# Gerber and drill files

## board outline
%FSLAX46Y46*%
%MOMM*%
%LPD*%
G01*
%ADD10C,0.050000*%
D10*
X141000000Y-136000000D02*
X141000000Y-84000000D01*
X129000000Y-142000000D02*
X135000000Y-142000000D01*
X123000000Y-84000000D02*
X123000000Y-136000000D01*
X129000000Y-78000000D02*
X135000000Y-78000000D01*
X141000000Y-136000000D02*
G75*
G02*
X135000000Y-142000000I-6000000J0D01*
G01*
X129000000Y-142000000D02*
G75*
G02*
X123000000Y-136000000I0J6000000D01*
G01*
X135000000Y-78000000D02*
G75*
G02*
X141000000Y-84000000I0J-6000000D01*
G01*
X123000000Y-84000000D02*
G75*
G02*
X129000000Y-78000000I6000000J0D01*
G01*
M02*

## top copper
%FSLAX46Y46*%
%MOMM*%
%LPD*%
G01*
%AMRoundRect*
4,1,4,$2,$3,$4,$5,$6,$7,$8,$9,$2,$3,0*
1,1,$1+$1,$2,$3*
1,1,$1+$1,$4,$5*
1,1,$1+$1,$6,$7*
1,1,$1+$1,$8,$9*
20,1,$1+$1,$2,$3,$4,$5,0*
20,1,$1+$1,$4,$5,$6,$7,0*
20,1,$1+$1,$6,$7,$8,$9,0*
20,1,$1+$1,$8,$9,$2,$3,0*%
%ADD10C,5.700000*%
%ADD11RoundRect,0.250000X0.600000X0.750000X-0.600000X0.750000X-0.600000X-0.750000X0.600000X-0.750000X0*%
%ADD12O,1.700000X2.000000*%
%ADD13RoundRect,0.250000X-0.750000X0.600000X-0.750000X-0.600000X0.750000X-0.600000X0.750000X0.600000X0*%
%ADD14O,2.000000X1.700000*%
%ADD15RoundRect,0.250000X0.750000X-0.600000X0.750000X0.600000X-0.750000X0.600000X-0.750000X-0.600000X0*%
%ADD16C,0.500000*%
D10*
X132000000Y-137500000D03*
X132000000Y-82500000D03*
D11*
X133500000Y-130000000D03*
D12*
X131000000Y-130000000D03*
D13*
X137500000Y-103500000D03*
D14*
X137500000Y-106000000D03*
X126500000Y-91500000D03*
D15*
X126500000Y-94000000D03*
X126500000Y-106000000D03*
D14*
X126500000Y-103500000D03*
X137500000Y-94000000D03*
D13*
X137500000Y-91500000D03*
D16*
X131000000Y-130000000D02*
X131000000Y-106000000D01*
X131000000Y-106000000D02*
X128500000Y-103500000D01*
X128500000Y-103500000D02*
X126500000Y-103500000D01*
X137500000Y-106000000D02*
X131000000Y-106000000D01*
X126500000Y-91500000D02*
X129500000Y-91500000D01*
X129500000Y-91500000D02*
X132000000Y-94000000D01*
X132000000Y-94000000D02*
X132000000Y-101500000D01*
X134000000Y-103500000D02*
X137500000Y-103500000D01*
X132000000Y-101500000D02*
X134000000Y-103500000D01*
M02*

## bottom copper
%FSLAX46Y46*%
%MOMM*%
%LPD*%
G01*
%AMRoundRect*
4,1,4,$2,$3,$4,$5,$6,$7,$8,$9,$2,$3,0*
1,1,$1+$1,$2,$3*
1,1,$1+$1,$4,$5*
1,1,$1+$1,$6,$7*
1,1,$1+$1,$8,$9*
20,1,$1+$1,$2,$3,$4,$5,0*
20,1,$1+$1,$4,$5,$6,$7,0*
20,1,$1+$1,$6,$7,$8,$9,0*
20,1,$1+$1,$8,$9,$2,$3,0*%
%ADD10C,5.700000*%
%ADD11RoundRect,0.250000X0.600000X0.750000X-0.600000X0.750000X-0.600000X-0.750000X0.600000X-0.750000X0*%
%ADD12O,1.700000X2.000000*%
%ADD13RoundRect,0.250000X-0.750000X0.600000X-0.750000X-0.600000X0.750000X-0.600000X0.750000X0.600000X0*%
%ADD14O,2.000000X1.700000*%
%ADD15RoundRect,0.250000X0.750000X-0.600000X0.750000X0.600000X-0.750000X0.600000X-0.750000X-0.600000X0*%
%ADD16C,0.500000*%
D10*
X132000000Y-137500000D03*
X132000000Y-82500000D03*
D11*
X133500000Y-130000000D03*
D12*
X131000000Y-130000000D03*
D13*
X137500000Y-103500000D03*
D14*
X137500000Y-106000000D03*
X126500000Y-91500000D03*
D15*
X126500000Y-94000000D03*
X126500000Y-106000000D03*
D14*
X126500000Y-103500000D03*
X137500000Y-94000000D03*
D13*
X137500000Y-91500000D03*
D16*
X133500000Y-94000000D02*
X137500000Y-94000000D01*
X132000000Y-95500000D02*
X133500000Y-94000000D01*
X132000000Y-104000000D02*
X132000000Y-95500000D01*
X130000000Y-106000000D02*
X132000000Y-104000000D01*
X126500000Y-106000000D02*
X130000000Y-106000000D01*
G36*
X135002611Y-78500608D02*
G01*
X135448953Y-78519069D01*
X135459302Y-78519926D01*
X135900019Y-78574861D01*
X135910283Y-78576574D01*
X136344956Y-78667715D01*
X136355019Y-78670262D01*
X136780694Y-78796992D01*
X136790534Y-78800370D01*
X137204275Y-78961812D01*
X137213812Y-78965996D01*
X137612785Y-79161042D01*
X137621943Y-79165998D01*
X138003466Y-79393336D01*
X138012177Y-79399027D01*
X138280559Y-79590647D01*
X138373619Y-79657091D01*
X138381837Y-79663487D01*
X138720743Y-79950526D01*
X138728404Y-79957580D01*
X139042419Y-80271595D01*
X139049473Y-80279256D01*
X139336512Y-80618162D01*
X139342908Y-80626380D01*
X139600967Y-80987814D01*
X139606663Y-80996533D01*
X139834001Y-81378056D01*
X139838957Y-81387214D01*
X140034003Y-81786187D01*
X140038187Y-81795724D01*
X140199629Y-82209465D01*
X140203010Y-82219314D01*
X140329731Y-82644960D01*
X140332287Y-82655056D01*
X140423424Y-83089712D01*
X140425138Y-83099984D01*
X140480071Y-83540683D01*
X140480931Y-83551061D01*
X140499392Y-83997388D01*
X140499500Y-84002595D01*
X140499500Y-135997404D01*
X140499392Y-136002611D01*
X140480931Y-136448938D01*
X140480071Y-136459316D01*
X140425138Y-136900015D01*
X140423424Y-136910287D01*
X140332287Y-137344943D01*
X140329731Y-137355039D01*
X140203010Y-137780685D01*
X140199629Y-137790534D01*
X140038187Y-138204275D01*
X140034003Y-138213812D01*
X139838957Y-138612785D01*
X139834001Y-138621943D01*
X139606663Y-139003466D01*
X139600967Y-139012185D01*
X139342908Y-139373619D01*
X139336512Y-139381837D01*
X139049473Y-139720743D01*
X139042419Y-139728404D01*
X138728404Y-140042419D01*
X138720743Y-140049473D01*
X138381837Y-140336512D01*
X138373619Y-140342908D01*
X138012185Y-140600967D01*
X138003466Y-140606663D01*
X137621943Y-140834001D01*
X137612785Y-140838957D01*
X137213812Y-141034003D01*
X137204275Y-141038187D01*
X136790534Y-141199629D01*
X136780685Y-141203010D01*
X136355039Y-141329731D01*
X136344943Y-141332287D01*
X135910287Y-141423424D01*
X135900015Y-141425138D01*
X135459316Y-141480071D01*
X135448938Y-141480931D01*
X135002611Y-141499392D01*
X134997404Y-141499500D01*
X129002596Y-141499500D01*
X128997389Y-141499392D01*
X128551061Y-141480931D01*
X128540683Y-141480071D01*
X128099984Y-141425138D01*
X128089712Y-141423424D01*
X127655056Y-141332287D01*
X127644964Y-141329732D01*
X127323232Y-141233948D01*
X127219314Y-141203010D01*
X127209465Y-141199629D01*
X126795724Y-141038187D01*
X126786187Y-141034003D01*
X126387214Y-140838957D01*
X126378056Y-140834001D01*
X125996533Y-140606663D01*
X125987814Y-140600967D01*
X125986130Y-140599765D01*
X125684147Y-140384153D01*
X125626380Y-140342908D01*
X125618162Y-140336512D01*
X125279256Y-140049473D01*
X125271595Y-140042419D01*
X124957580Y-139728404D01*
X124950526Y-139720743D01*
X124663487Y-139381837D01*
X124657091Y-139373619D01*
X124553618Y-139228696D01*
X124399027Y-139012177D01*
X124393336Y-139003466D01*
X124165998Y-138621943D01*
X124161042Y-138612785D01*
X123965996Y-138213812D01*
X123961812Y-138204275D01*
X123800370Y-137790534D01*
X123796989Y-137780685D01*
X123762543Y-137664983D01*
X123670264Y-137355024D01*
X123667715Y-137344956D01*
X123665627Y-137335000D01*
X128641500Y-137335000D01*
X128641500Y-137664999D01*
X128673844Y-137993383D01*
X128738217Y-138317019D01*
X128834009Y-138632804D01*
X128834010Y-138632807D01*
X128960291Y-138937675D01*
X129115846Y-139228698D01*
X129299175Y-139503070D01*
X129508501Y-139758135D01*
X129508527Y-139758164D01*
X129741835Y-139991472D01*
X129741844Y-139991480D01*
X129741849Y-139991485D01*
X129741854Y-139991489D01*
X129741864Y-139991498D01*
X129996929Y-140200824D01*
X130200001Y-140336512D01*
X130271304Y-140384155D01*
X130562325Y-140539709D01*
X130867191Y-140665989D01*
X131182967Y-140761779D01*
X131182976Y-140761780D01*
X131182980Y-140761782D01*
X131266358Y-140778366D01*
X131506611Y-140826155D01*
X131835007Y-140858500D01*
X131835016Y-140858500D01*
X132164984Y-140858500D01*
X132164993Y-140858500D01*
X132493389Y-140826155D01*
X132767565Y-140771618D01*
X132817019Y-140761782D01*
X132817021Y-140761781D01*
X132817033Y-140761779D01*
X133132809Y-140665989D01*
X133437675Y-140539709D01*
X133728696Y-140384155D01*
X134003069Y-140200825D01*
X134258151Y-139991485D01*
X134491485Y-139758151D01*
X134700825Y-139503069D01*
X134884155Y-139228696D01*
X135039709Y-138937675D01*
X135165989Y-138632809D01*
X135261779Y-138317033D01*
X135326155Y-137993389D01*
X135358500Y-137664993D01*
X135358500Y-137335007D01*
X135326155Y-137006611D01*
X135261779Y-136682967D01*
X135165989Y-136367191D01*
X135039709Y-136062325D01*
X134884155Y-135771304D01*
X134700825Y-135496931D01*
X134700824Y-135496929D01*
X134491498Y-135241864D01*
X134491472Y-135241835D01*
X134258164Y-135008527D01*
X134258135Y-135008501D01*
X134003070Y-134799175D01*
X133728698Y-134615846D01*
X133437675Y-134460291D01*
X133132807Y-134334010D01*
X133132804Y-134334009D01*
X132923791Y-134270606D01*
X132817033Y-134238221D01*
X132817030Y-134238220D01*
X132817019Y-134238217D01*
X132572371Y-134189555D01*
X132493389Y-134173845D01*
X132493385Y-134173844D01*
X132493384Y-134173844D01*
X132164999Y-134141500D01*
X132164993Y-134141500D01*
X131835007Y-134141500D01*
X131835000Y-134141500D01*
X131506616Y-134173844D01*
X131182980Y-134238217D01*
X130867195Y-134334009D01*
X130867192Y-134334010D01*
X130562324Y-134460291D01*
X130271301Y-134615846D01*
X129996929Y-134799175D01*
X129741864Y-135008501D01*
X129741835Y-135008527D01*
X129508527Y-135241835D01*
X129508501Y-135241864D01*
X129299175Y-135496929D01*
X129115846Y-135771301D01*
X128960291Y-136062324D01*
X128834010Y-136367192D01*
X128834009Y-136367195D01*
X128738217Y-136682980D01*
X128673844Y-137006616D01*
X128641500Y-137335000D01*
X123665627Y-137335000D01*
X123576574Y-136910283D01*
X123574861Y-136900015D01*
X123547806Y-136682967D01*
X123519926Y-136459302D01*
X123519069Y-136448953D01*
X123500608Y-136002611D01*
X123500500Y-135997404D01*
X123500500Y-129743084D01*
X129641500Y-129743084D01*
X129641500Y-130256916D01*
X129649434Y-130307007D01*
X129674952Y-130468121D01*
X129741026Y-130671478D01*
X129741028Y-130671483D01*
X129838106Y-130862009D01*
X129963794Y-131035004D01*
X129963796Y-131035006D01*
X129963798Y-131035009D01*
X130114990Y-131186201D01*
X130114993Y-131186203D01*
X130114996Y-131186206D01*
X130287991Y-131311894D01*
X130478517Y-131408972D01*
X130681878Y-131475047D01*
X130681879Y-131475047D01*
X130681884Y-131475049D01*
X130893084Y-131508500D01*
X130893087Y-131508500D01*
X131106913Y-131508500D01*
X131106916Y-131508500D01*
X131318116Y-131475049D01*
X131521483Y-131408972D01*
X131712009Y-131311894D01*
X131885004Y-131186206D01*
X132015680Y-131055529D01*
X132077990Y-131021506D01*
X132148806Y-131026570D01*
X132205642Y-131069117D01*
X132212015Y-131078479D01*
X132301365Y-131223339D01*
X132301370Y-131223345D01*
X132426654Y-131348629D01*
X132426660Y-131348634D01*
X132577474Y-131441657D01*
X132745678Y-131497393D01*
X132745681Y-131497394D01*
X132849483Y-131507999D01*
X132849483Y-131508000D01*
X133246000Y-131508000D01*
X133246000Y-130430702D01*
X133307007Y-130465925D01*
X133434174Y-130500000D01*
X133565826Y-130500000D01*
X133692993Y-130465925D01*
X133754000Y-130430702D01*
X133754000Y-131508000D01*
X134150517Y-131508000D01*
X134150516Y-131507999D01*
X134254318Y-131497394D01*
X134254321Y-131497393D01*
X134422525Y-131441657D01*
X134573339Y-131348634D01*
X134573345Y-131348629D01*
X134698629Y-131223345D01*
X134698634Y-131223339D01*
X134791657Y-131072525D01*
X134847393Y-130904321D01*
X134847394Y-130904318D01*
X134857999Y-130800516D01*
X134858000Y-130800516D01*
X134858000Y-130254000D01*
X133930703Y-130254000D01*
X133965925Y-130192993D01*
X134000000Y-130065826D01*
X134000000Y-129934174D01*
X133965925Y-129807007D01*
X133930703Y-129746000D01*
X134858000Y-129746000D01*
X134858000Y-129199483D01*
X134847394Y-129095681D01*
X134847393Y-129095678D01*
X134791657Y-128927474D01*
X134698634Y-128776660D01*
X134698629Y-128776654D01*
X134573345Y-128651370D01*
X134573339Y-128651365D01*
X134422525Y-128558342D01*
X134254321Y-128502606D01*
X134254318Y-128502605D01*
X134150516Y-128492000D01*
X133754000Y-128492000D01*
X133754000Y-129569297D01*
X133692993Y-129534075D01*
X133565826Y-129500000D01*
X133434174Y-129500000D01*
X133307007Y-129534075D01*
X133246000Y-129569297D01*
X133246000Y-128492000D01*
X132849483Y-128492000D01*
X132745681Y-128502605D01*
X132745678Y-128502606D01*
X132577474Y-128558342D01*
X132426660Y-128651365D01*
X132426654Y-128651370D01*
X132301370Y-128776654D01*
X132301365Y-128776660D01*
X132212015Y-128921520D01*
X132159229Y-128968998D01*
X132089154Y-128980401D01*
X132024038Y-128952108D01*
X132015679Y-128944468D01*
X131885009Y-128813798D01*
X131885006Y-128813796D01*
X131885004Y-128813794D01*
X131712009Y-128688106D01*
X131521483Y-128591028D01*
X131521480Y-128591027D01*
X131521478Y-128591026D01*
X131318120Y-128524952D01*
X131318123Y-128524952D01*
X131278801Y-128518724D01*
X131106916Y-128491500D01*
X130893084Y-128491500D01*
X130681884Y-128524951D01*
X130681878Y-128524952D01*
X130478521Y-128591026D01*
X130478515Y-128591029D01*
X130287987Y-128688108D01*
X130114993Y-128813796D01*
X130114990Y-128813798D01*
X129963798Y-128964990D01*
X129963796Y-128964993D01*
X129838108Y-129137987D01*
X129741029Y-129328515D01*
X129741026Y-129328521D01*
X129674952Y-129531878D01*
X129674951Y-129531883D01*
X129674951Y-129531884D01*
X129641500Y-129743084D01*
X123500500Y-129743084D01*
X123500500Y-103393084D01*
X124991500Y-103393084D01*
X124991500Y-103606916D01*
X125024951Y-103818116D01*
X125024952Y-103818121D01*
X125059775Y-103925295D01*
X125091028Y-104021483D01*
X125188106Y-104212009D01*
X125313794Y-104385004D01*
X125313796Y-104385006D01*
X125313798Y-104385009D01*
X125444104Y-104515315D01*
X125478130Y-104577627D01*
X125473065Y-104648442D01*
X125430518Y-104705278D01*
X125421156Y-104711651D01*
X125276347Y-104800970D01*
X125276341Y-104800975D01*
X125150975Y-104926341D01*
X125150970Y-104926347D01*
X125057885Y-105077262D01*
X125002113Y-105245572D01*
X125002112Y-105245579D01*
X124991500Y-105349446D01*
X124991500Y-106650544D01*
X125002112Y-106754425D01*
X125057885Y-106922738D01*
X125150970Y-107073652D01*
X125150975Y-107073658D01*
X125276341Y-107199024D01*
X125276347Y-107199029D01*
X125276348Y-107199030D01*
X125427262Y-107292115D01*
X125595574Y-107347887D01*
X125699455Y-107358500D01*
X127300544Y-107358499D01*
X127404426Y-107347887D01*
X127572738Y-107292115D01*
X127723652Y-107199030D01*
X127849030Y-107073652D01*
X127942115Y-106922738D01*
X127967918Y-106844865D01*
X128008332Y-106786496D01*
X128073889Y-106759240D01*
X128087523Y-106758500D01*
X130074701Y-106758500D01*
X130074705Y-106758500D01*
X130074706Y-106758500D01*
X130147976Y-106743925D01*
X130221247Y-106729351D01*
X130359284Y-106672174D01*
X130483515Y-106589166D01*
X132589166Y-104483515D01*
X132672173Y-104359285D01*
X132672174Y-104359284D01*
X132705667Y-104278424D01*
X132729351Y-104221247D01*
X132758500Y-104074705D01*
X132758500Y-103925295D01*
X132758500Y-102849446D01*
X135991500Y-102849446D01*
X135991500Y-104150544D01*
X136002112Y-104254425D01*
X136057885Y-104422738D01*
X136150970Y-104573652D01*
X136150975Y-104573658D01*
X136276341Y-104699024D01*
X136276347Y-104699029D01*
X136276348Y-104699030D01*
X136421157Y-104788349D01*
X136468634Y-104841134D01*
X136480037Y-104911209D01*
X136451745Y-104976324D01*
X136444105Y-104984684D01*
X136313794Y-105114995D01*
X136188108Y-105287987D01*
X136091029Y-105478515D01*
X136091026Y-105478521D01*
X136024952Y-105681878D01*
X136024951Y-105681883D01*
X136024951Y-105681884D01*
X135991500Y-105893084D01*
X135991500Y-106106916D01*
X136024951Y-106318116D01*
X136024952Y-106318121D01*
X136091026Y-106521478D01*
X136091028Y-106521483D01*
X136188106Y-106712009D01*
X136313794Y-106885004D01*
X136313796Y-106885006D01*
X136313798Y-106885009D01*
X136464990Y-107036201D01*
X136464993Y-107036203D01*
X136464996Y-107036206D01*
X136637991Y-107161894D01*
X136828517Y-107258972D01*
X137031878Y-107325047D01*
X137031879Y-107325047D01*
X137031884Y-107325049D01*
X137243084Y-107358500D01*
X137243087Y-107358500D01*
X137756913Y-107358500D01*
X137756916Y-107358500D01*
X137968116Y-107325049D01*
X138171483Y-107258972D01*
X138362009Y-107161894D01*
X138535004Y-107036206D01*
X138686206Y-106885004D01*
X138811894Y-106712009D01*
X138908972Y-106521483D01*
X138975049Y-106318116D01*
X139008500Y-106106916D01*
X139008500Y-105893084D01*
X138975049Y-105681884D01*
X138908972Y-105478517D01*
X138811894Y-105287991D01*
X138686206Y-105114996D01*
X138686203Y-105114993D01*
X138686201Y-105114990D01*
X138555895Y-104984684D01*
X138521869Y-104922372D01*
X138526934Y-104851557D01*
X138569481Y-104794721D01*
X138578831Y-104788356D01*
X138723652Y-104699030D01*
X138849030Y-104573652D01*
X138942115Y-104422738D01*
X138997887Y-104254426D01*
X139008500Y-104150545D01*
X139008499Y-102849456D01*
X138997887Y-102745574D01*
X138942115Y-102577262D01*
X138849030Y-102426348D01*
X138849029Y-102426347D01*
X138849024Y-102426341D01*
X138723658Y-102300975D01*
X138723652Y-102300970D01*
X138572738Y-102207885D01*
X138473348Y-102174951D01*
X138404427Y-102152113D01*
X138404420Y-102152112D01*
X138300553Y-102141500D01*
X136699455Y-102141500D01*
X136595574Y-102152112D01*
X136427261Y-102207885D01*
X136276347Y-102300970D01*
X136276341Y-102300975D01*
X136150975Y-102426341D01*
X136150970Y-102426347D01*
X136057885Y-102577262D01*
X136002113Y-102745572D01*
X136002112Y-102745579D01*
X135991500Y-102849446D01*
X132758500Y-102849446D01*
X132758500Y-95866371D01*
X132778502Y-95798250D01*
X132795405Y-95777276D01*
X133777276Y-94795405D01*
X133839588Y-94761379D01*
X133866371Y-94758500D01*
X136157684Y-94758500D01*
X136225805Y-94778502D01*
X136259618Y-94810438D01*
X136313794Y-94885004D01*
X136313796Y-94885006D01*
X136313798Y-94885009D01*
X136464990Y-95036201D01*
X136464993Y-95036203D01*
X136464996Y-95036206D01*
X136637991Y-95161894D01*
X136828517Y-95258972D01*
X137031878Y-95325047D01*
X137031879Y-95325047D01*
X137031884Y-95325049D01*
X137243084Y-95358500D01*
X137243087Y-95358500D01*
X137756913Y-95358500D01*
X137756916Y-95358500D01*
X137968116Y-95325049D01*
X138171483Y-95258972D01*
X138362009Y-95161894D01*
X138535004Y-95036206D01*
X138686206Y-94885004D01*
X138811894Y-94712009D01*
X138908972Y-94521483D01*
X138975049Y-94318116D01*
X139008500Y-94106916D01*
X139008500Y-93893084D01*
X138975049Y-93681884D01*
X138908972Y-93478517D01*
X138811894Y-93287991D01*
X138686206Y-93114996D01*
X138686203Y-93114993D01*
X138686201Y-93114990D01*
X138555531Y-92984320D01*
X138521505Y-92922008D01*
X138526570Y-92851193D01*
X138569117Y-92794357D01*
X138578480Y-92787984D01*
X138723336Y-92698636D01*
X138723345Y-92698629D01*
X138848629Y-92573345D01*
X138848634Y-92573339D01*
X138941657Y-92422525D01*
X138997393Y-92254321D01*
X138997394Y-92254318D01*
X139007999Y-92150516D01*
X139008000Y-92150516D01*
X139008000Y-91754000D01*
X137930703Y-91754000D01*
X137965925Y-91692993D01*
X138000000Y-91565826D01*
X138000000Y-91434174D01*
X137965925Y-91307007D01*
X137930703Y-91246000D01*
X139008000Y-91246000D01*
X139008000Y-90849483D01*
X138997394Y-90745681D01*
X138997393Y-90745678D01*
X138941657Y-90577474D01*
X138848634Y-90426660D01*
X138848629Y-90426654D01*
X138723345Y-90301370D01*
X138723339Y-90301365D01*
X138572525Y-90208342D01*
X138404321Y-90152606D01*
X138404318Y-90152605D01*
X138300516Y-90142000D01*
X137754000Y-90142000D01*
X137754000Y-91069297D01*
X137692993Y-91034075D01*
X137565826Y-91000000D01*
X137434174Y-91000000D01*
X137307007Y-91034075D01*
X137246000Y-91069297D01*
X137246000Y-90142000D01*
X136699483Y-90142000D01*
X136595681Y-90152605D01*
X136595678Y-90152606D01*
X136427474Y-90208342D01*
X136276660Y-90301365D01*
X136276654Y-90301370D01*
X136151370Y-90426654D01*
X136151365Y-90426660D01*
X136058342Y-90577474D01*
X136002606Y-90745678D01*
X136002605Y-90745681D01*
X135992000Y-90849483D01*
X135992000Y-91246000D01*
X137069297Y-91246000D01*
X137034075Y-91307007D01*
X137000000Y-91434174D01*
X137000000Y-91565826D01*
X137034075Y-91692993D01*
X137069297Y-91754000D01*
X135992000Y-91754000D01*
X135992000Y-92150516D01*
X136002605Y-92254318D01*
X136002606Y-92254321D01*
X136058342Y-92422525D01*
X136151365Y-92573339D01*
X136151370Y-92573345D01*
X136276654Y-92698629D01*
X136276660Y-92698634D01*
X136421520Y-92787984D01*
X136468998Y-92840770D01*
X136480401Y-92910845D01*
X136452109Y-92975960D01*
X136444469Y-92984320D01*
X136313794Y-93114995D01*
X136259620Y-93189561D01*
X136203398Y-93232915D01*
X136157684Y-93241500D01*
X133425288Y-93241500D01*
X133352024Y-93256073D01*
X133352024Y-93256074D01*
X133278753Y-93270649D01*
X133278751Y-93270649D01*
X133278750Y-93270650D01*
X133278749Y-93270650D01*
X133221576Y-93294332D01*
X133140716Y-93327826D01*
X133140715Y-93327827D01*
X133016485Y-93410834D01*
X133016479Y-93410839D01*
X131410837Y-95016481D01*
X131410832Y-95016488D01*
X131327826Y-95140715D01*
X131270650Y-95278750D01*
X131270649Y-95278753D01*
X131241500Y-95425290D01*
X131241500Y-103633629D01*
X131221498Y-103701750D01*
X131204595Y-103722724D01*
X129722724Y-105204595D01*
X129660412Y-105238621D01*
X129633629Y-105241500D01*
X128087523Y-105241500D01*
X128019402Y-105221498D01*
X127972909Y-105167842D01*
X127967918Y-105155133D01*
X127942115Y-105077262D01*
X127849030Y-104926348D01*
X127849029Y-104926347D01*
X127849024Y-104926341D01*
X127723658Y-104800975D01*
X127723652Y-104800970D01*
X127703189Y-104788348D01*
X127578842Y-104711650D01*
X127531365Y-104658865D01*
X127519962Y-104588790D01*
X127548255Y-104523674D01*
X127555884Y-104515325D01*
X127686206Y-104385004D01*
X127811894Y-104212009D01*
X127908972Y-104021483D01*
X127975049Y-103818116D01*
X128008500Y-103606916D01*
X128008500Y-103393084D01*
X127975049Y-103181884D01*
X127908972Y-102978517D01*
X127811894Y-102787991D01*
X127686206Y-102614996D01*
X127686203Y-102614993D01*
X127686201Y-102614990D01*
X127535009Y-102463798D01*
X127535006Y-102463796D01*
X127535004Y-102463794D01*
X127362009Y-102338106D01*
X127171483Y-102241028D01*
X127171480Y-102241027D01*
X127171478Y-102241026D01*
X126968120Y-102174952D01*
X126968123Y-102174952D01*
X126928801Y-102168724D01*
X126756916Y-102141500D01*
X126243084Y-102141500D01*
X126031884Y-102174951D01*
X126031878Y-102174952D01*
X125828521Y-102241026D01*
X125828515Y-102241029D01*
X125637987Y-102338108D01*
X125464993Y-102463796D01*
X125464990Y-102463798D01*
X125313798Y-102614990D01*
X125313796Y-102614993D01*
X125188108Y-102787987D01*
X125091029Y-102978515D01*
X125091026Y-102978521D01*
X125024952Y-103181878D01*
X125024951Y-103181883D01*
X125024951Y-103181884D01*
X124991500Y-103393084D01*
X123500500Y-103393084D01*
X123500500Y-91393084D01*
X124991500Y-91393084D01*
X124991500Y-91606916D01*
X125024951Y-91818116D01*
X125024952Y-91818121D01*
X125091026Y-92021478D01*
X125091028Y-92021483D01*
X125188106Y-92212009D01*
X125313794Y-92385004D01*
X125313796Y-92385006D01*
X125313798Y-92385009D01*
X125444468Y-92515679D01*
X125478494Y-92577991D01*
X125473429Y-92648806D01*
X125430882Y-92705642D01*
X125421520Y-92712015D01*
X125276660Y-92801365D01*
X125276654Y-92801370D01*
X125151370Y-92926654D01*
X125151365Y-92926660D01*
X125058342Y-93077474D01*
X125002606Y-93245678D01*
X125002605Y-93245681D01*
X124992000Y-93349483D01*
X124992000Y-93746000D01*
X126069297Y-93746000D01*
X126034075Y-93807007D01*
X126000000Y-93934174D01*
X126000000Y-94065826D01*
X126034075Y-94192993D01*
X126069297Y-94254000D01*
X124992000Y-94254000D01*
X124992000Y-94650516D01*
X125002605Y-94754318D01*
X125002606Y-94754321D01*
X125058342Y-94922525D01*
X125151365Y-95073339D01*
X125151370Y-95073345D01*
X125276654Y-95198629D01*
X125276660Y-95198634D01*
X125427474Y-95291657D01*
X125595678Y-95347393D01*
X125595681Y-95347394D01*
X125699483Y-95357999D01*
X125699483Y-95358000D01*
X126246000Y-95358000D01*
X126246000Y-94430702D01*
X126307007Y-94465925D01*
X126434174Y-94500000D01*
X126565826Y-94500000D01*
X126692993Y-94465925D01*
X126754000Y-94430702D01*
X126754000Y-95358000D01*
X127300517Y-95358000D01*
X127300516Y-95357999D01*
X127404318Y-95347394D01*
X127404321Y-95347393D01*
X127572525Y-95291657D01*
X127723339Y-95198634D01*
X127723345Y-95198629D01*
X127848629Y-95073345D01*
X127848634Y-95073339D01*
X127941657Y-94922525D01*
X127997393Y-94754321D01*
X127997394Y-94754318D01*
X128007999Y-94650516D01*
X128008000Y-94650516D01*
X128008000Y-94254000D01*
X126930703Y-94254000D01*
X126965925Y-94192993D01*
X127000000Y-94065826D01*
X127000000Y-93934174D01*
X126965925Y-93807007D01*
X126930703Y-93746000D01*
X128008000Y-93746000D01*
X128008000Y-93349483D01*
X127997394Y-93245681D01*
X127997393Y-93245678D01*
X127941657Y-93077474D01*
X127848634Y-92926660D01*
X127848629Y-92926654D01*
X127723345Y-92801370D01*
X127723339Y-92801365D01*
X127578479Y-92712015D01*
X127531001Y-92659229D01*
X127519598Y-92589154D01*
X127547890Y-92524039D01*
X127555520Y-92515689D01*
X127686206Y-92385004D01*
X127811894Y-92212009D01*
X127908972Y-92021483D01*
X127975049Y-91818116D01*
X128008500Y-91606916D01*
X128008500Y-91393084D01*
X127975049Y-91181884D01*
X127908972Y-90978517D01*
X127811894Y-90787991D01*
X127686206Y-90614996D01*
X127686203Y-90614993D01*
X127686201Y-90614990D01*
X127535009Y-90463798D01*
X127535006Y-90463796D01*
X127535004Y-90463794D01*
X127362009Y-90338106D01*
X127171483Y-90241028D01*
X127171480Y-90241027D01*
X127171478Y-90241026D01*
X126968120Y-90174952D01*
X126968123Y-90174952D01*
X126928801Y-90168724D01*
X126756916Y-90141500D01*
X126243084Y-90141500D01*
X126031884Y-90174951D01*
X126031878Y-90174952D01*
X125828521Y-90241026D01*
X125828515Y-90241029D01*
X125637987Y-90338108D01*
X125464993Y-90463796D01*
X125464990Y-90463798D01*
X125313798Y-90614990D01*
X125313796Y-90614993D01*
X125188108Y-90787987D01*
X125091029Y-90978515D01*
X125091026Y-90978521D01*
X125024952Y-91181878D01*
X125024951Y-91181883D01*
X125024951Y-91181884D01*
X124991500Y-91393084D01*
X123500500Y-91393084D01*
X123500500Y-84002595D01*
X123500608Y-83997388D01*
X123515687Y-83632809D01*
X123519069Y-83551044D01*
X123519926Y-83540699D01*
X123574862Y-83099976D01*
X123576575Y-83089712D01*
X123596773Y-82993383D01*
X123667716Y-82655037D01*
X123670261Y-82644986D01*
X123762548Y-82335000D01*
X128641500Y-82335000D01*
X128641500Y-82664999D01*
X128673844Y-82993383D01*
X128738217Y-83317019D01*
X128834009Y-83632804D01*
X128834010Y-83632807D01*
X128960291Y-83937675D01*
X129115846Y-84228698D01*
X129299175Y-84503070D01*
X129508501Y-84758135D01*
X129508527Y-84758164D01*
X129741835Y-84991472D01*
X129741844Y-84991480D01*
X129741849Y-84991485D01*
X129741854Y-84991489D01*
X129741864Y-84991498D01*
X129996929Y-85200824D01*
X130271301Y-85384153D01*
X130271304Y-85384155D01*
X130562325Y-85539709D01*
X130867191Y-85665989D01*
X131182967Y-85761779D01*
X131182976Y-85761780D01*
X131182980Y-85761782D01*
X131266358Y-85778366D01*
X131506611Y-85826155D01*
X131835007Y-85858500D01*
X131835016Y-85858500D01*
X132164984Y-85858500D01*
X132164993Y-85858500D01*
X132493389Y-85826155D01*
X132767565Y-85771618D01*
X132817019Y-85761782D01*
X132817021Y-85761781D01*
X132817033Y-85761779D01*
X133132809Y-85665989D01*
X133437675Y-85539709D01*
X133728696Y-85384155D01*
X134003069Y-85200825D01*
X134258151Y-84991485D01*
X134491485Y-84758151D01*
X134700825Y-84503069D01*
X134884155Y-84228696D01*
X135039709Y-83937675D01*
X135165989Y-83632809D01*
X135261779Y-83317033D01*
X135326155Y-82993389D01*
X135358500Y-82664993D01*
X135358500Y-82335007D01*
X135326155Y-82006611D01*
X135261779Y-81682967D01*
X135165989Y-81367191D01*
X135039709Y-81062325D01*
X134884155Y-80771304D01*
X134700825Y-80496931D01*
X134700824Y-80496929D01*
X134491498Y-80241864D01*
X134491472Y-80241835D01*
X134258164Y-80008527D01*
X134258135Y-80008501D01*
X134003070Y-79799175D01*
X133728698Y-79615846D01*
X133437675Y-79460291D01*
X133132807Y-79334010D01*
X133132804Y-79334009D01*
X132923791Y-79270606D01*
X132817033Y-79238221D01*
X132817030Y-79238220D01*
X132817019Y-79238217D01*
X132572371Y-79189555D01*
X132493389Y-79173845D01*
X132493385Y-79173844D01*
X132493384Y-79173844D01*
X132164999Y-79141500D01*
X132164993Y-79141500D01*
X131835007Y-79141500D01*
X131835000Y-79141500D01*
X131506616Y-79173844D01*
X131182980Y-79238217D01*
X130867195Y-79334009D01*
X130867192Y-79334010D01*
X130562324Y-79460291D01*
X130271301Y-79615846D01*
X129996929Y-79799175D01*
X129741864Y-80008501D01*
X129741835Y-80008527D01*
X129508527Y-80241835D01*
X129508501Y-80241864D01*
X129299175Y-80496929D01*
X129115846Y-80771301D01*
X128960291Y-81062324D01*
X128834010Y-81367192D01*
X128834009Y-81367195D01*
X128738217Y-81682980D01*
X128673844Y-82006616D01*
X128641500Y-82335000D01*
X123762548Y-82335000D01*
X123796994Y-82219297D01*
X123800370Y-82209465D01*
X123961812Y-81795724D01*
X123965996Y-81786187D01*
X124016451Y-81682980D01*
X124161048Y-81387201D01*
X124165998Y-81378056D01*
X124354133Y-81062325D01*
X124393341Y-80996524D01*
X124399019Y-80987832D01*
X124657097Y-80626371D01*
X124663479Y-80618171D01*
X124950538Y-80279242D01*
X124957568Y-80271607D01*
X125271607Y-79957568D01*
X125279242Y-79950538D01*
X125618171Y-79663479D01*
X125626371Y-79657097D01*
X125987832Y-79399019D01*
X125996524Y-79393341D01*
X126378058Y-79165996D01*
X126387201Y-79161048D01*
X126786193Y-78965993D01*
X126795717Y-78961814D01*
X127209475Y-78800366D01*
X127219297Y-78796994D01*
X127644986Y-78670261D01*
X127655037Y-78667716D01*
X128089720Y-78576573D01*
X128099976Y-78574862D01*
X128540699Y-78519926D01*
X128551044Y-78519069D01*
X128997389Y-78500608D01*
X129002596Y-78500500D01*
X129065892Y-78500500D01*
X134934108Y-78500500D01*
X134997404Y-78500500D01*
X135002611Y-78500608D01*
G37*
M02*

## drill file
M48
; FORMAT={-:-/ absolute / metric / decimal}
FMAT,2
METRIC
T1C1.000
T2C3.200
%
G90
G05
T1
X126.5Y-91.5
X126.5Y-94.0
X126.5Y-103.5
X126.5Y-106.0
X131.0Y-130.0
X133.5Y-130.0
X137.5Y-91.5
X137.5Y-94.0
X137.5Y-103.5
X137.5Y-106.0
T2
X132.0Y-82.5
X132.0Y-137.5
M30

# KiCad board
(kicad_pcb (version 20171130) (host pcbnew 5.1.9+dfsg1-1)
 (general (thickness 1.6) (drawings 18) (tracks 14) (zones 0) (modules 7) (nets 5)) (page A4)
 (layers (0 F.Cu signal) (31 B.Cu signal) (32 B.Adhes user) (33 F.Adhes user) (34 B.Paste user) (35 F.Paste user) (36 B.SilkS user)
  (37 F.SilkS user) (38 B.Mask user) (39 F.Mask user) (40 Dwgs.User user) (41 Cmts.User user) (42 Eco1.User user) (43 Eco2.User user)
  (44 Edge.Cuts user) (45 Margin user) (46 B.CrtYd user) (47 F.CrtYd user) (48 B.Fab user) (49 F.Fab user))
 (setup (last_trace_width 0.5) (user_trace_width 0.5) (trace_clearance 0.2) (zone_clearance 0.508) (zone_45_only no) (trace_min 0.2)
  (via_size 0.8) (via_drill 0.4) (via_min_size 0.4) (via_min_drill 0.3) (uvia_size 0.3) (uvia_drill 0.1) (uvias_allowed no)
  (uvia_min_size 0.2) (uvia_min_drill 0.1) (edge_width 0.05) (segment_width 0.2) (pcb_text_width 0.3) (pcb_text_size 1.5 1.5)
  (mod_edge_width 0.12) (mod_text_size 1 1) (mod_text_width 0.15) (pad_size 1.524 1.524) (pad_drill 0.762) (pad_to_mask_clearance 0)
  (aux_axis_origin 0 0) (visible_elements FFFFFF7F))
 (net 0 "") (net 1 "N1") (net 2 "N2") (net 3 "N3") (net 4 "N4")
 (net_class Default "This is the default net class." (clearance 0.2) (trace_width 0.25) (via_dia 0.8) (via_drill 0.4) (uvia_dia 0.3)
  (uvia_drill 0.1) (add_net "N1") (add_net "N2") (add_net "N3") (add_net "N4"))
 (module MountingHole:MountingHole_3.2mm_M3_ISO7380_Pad (layer F.Cu) (at 132 137.5)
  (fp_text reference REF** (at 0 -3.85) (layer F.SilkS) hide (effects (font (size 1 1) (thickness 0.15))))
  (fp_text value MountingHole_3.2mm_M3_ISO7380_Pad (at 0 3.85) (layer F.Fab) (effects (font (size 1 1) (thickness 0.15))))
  (pad 1 thru_hole circle (at 0 0) (size 5.7 5.7) (drill 3.2) (layers *.Cu *.Mask)))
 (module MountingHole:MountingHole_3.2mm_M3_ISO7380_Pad (layer F.Cu) (at 132 82.5)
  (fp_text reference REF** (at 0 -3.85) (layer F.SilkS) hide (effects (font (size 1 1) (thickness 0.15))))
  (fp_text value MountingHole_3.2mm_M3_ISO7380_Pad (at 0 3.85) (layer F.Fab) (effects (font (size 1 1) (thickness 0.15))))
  (pad 1 thru_hole circle (at 0 0) (size 5.7 5.7) (drill 3.2) (layers *.Cu *.Mask)))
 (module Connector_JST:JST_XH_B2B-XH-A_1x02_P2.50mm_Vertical (layer F.Cu) (at 133.5 130 180)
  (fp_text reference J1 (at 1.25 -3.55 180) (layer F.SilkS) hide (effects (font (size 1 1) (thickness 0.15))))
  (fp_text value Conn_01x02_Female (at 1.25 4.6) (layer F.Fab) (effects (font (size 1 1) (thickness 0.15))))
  (pad 1 thru_hole roundrect (at 0 0 180) (size 1.7 2) (drill 1) (layers *.Cu *.Mask) (roundrect_rratio 0.1470588235294118) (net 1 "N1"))
  (pad 2 thru_hole oval (at 2.5 0 180) (size 1.7 2) (drill 1) (layers *.Cu *.Mask) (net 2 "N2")))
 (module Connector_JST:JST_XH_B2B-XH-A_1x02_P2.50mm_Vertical (layer F.Cu) (at 137.5 103.5 270)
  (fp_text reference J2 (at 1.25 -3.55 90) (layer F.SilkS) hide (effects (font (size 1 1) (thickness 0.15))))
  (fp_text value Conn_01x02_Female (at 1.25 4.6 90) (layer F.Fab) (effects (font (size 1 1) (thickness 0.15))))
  (pad 1 thru_hole roundrect (at 0 0 270) (size 1.7 2) (drill 1) (layers *.Cu *.Mask) (roundrect_rratio 0.1470588235294118) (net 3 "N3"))
  (pad 2 thru_hole oval (at 2.5 0 270) (size 1.7 2) (drill 1) (layers *.Cu *.Mask) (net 2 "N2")))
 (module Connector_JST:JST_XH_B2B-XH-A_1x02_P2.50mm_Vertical (layer F.Cu) (at 126.5 94 90)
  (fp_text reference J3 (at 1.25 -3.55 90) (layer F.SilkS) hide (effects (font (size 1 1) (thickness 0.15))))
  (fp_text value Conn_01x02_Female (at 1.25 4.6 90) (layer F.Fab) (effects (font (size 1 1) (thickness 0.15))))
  (pad 2 thru_hole oval (at 2.5 0 90) (size 1.7 2) (drill 1) (layers *.Cu *.Mask) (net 3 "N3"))
  (pad 1 thru_hole roundrect (at 0 0 90) (size 1.7 2) (drill 1) (layers *.Cu *.Mask) (roundrect_rratio 0.1470588235294118) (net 1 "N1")))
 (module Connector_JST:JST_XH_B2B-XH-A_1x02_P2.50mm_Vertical (layer F.Cu) (at 126.5 106 90)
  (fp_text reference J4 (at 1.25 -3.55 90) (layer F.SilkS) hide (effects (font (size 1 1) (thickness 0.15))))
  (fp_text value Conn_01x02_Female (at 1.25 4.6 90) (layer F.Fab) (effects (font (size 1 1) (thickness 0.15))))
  (pad 1 thru_hole roundrect (at 0 0 90) (size 1.7 2) (drill 1) (layers *.Cu *.Mask) (roundrect_rratio 0.1470588235294118) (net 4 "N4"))
  (pad 2 thru_hole oval (at 2.5 0 90) (size 1.7 2) (drill 1) (layers *.Cu *.Mask) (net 2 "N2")))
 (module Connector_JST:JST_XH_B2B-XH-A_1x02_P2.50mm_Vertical (layer F.Cu) (at 137.5 91.5 270)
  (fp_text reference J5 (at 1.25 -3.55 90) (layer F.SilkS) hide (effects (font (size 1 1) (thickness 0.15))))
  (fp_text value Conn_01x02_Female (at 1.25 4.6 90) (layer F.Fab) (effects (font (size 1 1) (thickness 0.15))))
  (pad 2 thru_hole oval (at 2.5 0 270) (size 1.7 2) (drill 1) (layers *.Cu *.Mask) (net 4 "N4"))
  (pad 1 thru_hole roundrect (at 0 0 270) (size 1.7 2) (drill 1) (layers *.Cu *.Mask) (roundrect_rratio 0.1470588235294118) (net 1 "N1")))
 (gr_line (start 141 136) (end 141 84) (layer Edge.Cuts) (width 0.05))
 (gr_line (start 129 142) (end 135 142) (layer Edge.Cuts) (width 0.05))
 (gr_line (start 123 84) (end 123 136) (layer Edge.Cuts) (width 0.05))
 (gr_line (start 129 78) (end 135 78) (layer Edge.Cuts) (width 0.05))
 (gr_arc (start 135 136) (end 135 142) (angle -90) (layer Edge.Cuts) (width 0.05))
 (gr_arc (start 129 136) (end 123 136) (angle -90) (layer Edge.Cuts) (width 0.05))
 (gr_arc (start 135 84) (end 141 84) (angle -90) (layer Edge.Cuts) (width 0.05))
 (gr_arc (start 129 84) (end 129 78) (angle -90) (layer Edge.Cuts) (width 0.05))
 (segment (start 131 130) (end 131 106) (width 0.5) (layer F.Cu) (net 2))
 (segment (start 131 106) (end 128.5 103.5) (width 0.5) (layer F.Cu) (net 2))
 (segment (start 128.5 103.5) (end 126.5 103.5) (width 0.5) (layer F.Cu) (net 2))
 (segment (start 137.5 106) (end 131 106) (width 0.5) (layer F.Cu) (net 2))
 (segment (start 126.5 91.5) (end 129.5 91.5) (width 0.5) (layer F.Cu) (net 3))
 (segment (start 129.5 91.5) (end 132 94) (width 0.5) (layer F.Cu) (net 3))
 (segment (start 132 94) (end 132 101.5) (width 0.5) (layer F.Cu) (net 3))
 (segment (start 134 103.5) (end 137.5 103.5) (width 0.5) (layer F.Cu) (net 3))
 (segment (start 132 101.5) (end 134 103.5) (width 0.5) (layer F.Cu) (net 3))
 (segment (start 133.5 94) (end 137.5 94) (width 0.5) (layer B.Cu) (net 4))
 (segment (start 132 95.5) (end 133.5 94) (width 0.5) (layer B.Cu) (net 4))
 (segment (start 132 104) (end 132 95.5) (width 0.5) (layer B.Cu) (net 4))
 (segment (start 130 106) (end 132 104) (width 0.5) (layer B.Cu) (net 4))
 (segment (start 126.5 106) (end 130 106) (width 0.5) (layer B.Cu) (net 4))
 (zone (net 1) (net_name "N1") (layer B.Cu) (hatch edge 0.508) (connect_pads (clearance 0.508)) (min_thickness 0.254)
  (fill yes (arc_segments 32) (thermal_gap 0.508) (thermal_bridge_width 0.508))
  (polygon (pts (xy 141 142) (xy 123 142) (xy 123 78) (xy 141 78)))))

